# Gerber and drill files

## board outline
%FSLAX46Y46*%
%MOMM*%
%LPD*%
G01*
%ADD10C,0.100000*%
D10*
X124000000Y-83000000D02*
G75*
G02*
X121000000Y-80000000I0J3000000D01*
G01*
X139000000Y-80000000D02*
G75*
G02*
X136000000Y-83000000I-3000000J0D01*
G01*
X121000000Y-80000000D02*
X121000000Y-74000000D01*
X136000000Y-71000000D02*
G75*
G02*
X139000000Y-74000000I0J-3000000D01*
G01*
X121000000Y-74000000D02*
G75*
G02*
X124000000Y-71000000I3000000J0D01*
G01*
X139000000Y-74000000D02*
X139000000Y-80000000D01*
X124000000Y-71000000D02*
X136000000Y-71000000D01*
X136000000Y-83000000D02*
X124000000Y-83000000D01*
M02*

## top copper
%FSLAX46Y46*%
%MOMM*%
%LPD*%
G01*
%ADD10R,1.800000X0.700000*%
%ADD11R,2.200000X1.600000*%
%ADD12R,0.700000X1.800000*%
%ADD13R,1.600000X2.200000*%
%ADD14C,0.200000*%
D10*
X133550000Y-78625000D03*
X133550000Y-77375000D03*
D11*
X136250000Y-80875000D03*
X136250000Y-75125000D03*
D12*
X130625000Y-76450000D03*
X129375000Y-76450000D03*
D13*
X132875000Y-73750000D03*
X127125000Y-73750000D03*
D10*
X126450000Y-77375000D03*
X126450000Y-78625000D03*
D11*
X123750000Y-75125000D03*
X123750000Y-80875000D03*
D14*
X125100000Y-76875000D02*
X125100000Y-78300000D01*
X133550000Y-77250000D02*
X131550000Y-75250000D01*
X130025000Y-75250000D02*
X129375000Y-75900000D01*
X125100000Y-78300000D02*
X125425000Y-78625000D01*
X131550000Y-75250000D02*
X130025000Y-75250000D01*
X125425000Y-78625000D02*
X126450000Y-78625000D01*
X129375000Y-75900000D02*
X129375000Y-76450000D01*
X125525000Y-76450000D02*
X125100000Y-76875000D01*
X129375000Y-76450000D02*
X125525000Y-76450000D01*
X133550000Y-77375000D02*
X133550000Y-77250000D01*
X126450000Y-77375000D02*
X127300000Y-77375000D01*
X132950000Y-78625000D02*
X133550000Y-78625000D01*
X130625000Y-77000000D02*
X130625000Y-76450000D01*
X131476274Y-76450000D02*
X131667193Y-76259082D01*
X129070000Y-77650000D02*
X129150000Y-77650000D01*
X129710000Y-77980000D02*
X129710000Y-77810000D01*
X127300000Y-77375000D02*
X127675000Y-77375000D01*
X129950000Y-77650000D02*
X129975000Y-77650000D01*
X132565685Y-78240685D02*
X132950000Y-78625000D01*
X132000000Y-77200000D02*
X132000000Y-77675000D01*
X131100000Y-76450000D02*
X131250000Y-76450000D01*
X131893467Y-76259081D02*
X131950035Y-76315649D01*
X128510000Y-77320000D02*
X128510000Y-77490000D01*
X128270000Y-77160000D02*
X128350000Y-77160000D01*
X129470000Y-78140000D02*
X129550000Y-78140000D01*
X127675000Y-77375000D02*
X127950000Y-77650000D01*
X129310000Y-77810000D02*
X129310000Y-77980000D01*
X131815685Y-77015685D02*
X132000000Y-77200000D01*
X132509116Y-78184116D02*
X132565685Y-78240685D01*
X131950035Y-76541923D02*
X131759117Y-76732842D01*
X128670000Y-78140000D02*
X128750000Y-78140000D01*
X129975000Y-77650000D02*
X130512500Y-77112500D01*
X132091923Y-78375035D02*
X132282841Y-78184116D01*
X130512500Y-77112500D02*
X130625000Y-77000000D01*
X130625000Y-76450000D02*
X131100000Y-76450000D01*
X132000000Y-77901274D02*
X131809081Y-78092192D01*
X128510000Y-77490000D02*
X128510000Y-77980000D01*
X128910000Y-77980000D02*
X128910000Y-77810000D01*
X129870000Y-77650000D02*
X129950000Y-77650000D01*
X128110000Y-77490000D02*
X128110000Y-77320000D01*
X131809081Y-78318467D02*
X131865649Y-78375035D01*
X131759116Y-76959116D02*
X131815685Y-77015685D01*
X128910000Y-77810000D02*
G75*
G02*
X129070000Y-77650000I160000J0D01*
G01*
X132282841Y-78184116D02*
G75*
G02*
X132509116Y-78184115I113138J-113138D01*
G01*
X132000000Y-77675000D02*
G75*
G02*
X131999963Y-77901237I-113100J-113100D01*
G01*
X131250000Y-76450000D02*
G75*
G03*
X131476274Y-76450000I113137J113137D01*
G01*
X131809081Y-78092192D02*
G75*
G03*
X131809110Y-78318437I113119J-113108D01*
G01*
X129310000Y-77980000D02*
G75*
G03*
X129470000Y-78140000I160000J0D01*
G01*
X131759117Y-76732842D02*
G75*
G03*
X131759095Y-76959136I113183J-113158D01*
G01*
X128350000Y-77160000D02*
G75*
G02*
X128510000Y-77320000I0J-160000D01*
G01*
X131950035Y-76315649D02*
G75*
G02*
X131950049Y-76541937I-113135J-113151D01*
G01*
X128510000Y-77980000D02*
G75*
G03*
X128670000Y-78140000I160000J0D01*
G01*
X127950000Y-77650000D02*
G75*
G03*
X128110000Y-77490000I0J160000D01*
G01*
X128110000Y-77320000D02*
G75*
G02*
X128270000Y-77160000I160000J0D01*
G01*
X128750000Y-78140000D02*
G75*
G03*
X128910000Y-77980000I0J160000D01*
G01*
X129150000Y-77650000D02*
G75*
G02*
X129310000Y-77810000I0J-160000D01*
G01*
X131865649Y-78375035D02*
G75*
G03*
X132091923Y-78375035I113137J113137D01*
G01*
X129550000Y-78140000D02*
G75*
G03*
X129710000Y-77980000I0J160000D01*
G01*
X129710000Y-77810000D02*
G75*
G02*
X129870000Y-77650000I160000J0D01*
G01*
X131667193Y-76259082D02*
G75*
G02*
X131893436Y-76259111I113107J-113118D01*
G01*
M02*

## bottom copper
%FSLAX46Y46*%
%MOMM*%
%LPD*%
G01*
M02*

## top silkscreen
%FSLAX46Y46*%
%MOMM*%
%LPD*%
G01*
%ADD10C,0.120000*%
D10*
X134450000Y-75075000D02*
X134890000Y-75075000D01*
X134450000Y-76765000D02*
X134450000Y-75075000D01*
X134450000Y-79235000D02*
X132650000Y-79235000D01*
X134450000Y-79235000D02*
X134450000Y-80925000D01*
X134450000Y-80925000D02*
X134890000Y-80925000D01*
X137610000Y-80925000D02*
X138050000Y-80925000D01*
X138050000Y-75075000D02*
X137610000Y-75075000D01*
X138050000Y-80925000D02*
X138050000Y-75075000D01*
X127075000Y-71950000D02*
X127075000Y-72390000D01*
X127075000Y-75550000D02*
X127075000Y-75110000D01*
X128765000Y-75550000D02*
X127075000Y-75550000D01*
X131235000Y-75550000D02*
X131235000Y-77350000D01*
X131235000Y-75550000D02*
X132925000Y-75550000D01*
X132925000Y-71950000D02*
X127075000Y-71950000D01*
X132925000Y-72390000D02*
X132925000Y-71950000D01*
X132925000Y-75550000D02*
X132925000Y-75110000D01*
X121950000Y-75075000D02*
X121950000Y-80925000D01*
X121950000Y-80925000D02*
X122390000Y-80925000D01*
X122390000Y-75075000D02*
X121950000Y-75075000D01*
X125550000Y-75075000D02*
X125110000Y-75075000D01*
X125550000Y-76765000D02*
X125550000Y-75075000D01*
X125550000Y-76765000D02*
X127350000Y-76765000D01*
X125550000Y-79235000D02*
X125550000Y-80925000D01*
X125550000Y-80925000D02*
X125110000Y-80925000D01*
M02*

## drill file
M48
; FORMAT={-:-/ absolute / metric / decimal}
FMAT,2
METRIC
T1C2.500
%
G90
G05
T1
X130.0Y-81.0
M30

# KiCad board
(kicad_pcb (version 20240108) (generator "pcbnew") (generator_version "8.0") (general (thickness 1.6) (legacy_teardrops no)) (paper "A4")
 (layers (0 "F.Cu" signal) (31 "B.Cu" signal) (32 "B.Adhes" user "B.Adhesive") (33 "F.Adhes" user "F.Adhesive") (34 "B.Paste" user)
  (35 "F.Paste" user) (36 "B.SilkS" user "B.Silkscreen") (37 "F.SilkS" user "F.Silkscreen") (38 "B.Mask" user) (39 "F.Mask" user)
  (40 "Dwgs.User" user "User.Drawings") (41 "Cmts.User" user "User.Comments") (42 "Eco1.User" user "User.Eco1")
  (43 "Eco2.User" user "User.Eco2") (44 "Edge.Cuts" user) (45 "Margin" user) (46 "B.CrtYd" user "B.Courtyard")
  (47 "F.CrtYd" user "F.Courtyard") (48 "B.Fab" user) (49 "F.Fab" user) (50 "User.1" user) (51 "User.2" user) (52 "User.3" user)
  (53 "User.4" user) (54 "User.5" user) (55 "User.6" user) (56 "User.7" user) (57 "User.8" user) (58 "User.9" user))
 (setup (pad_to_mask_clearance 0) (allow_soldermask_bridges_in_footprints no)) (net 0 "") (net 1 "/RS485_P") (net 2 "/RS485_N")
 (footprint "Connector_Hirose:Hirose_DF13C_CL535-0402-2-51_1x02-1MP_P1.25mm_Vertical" (layer "F.Cu") (at 135 78 90)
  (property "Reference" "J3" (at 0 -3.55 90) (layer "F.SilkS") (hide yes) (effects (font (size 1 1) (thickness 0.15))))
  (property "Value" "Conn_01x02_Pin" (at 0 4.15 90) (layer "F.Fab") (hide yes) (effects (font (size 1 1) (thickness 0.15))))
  (fp_line (start 2.925 -0.55) (end 2.925 -0.11) (stroke (width 0.12) (type solid)) (layer "F.SilkS"))
  (fp_line (start 1.235 -0.55) (end 2.925 -0.55) (stroke (width 0.12) (type solid)) (layer "F.SilkS"))
  (fp_line (start -1.235 -0.55) (end -1.235 -2.35) (stroke (width 0.12) (type solid)) (layer "F.SilkS"))
  (fp_line (start -1.235 -0.55) (end -2.925 -0.55) (stroke (width 0.12) (type solid)) (layer "F.SilkS"))
  (fp_line (start -2.925 -0.55) (end -2.925 -0.11) (stroke (width 0.12) (type solid)) (layer "F.SilkS"))
  (fp_line (start -2.925 2.61) (end -2.925 3.05) (stroke (width 0.12) (type solid)) (layer "F.SilkS"))
  (fp_line (start 2.925 3.05) (end 2.925 2.61) (stroke (width 0.12) (type solid)) (layer "F.SilkS"))
  (fp_line (start -2.925 3.05) (end 2.925 3.05) (stroke (width 0.12) (type solid)) (layer "F.SilkS"))
  (pad "1" smd rect (at -0.625 -1.45 90) (size 0.7 1.8) (layers "F.Cu" "F.Paste" "F.Mask") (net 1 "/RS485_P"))
  (pad "2" smd rect (at 0.625 -1.45 90) (size 0.7 1.8) (layers "F.Cu" "F.Paste" "F.Mask") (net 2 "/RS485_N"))
  (pad "MP" smd rect (at -2.875 1.25 90) (size 1.6 2.2) (layers "F.Cu" "F.Paste" "F.Mask"))
  (pad "MP" smd rect (at 2.875 1.25 90) (size 1.6 2.2) (layers "F.Cu" "F.Paste" "F.Mask")))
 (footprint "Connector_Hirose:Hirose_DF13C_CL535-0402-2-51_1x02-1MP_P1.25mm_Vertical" (layer "F.Cu") (at 130 75 180)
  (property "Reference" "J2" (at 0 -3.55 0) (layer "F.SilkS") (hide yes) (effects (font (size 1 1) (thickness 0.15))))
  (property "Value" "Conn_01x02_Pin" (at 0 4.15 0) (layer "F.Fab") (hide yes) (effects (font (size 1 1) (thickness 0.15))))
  (fp_line (start 2.925 3.05) (end 2.925 2.61) (stroke (width 0.12) (type solid)) (layer "F.SilkS"))
  (fp_line (start 2.925 -0.55) (end 2.925 -0.11) (stroke (width 0.12) (type solid)) (layer "F.SilkS"))
  (fp_line (start 1.235 -0.55) (end 2.925 -0.55) (stroke (width 0.12) (type solid)) (layer "F.SilkS"))
  (fp_line (start -1.235 -0.55) (end -1.235 -2.35) (stroke (width 0.12) (type solid)) (layer "F.SilkS"))
  (fp_line (start -1.235 -0.55) (end -2.925 -0.55) (stroke (width 0.12) (type solid)) (layer "F.SilkS"))
  (fp_line (start -2.925 3.05) (end 2.925 3.05) (stroke (width 0.12) (type solid)) (layer "F.SilkS"))
  (fp_line (start -2.925 2.61) (end -2.925 3.05) (stroke (width 0.12) (type solid)) (layer "F.SilkS"))
  (fp_line (start -2.925 -0.55) (end -2.925 -0.11) (stroke (width 0.12) (type solid)) (layer "F.SilkS"))
  (pad "1" smd rect (at -0.625 -1.45 180) (size 0.7 1.8) (layers "F.Cu" "F.Paste" "F.Mask") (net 1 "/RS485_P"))
  (pad "2" smd rect (at 0.625 -1.45 180) (size 0.7 1.8) (layers "F.Cu" "F.Paste" "F.Mask") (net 2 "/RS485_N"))
  (pad "MP" smd rect (at -2.875 1.25 180) (size 1.6 2.2) (layers "F.Cu" "F.Paste" "F.Mask"))
  (pad "MP" smd rect (at 2.875 1.25 180) (size 1.6 2.2) (layers "F.Cu" "F.Paste" "F.Mask")))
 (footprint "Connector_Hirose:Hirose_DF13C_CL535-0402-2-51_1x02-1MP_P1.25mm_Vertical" (layer "F.Cu") (at 125 78 -90)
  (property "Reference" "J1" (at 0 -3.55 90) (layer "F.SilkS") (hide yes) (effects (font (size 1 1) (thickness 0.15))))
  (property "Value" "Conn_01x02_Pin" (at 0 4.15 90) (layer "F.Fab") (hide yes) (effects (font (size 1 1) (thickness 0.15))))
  (fp_line (start -2.925 3.05) (end 2.925 3.05) (stroke (width 0.12) (type solid)) (layer "F.SilkS"))
  (fp_line (start 2.925 3.05) (end 2.925 2.61) (stroke (width 0.12) (type solid)) (layer "F.SilkS"))
  (fp_line (start -2.925 2.61) (end -2.925 3.05) (stroke (width 0.12) (type solid)) (layer "F.SilkS"))
  (fp_line (start -2.925 -0.55) (end -2.925 -0.11) (stroke (width 0.12) (type solid)) (layer "F.SilkS"))
  (fp_line (start -1.235 -0.55) (end -2.925 -0.55) (stroke (width 0.12) (type solid)) (layer "F.SilkS"))
  (fp_line (start -1.235 -0.55) (end -1.235 -2.35) (stroke (width 0.12) (type solid)) (layer "F.SilkS"))
  (fp_line (start 1.235 -0.55) (end 2.925 -0.55) (stroke (width 0.12) (type solid)) (layer "F.SilkS"))
  (fp_line (start 2.925 -0.55) (end 2.925 -0.11) (stroke (width 0.12) (type solid)) (layer "F.SilkS"))
  (pad "1" smd rect (at -0.625 -1.45 270) (size 0.7 1.8) (layers "F.Cu" "F.Paste" "F.Mask") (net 1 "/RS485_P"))
  (pad "2" smd rect (at 0.625 -1.45 270) (size 0.7 1.8) (layers "F.Cu" "F.Paste" "F.Mask") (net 2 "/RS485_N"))
  (pad "MP" smd rect (at -2.875 1.25 270) (size 1.6 2.2) (layers "F.Cu" "F.Paste" "F.Mask"))
  (pad "MP" smd rect (at 2.875 1.25 270) (size 1.6 2.2) (layers "F.Cu" "F.Paste" "F.Mask")))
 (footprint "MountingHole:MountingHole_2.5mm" (layer "F.Cu") (at 130 81)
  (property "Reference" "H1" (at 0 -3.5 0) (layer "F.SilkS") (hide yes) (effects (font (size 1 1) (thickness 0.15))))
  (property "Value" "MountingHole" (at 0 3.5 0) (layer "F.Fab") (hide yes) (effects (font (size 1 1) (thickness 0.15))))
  (pad "" np_thru_hole circle (at 0 0) (size 2.5 2.5) (drill 2.5) (layers "*.Cu" "*.Mask")))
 (gr_arc (start 124 83) (mid 121.87868 82.12132) (end 121 80) (stroke (width 0.1) (type default)) (layer "Edge.Cuts"))
 (gr_arc (start 139 80) (mid 138.12132 82.12132) (end 136 83) (stroke (width 0.1) (type default)) (layer "Edge.Cuts"))
 (gr_line (start 121 80) (end 121 74) (stroke (width 0.1) (type default)) (layer "Edge.Cuts"))
 (gr_arc (start 136 71) (mid 138.12132 71.87868) (end 139 74) (stroke (width 0.1) (type default)) (layer "Edge.Cuts"))
 (gr_arc (start 121 74) (mid 121.87868 71.87868) (end 124 71) (stroke (width 0.1) (type default)) (layer "Edge.Cuts"))
 (gr_line (start 139 74) (end 139 80) (stroke (width 0.1) (type default)) (layer "Edge.Cuts"))
 (gr_line (start 124 71) (end 136 71) (stroke (width 0.1) (type default)) (layer "Edge.Cuts"))
 (gr_line (start 136 83) (end 124 83) (stroke (width 0.1) (type default)) (layer "Edge.Cuts"))
 (segment (start 125.1 76.875) (end 125.1 78.3) (width 0.2) (layer "F.Cu") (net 2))
 (segment (start 133.55 77.25) (end 131.55 75.25) (width 0.2) (layer "F.Cu") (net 2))
 (segment (start 130.025 75.25) (end 129.375 75.9) (width 0.2) (layer "F.Cu") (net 2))
 (segment (start 125.1 78.3) (end 125.425 78.625) (width 0.2) (layer "F.Cu") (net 2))
 (segment (start 131.55 75.25) (end 130.025 75.25) (width 0.2) (layer "F.Cu") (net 2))
 (segment (start 125.425 78.625) (end 126.45 78.625) (width 0.2) (layer "F.Cu") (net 2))
 (segment (start 129.375 75.9) (end 129.375 76.45) (width 0.2) (layer "F.Cu") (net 2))
 (segment (start 125.525 76.45) (end 125.1 76.875) (width 0.2) (layer "F.Cu") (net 2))
 (segment (start 129.375 76.45) (end 125.525 76.45) (width 0.2) (layer "F.Cu") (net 2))
 (segment (start 133.55 77.375) (end 133.55 77.25) (width 0.2) (layer "F.Cu") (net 2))
 (segment (start 126.45 77.375) (end 127.3 77.375) (width 0.2) (layer "F.Cu") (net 1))
 (segment (start 132.95 78.625) (end 133.55 78.625) (width 0.2) (layer "F.Cu") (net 1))
 (segment (start 130.625 77) (end 130.625 76.45) (width 0.2) (layer "F.Cu") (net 1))
 (segment (start 131.476274 76.45) (end 131.667193 76.259082) (width 0.2) (layer "F.Cu") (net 1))
 (segment (start 129.07 77.65) (end 129.15 77.65) (width 0.2) (layer "F.Cu") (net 1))
 (segment (start 129.71 77.98) (end 129.71 77.81) (width 0.2) (layer "F.Cu") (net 1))
 (segment (start 127.3 77.375) (end 127.675 77.375) (width 0.2) (layer "F.Cu") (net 1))
 (segment (start 129.95 77.65) (end 129.975 77.65) (width 0.2) (layer "F.Cu") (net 1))
 (segment (start 132.565685 78.240685) (end 132.95 78.625) (width 0.2) (layer "F.Cu") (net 1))
 (segment (start 132 77.2) (end 132 77.675) (width 0.2) (layer "F.Cu") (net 1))
 (segment (start 131.1 76.45) (end 131.25 76.45) (width 0.2) (layer "F.Cu") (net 1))
 (segment (start 131.893467 76.259081) (end 131.950035 76.315649) (width 0.2) (layer "F.Cu") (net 1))
 (segment (start 128.51 77.32) (end 128.51 77.49) (width 0.2) (layer "F.Cu") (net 1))
 (segment (start 128.27 77.16) (end 128.35 77.16) (width 0.2) (layer "F.Cu") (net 1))
 (segment (start 129.47 78.14) (end 129.55 78.14) (width 0.2) (layer "F.Cu") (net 1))
 (segment (start 127.675 77.375) (end 127.95 77.65) (width 0.2) (layer "F.Cu") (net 1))
 (segment (start 129.31 77.81) (end 129.31 77.98) (width 0.2) (layer "F.Cu") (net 1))
 (segment (start 131.815685 77.015685) (end 132 77.2) (width 0.2) (layer "F.Cu") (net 1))
 (segment (start 132.509116 78.184116) (end 132.565685 78.240685) (width 0.2) (layer "F.Cu") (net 1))
 (segment (start 131.950035 76.541923) (end 131.759117 76.732842) (width 0.2) (layer "F.Cu") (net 1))
 (segment (start 128.67 78.14) (end 128.75 78.14) (width 0.2) (layer "F.Cu") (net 1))
 (segment (start 129.975 77.65) (end 130.5125 77.1125) (width 0.2) (layer "F.Cu") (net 1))
 (segment (start 132.091923 78.375035) (end 132.282841 78.184116) (width 0.2) (layer "F.Cu") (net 1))
 (segment (start 130.5125 77.1125) (end 130.625 77) (width 0.2) (layer "F.Cu") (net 1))
 (segment (start 130.625 76.45) (end 131.1 76.45) (width 0.2) (layer "F.Cu") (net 1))
 (segment (start 132 77.901274) (end 131.809081 78.092192) (width 0.2) (layer "F.Cu") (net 1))
 (segment (start 128.51 77.49) (end 128.51 77.98) (width 0.2) (layer "F.Cu") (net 1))
 (segment (start 128.91 77.98) (end 128.91 77.81) (width 0.2) (layer "F.Cu") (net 1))
 (segment (start 129.87 77.65) (end 129.95 77.65) (width 0.2) (layer "F.Cu") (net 1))
 (segment (start 128.11 77.49) (end 128.11 77.32) (width 0.2) (layer "F.Cu") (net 1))
 (segment (start 131.809081 78.318467) (end 131.865649 78.375035) (width 0.2) (layer "F.Cu") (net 1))
 (segment (start 131.759116 76.959116) (end 131.815685 77.015685) (width 0.2) (layer "F.Cu") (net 1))
 (arc (start 128.91 77.81) (mid 128.956863 77.696863) (end 129.07 77.65) (width 0.2) (layer "F.Cu") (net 1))
 (arc (start 132.282841 78.184116) (mid 132.395978 78.137253) (end 132.509116 78.184116) (width 0.2) (layer "F.Cu") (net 1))
 (arc (start 132 77.675) (mid 132.046863 77.788137) (end 132 77.901274) (width 0.2) (layer "F.Cu") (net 1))
 (arc (start 131.25 76.45) (mid 131.363137 76.496863) (end 131.476274 76.45) (width 0.2) (layer "F.Cu") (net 1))
 (arc (start 131.809081 78.092192) (mid 131.762218 78.205329) (end 131.809081 78.318467) (width 0.2) (layer "F.Cu") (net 1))
 (arc (start 129.31 77.98) (mid 129.356863 78.093137) (end 129.47 78.14) (width 0.2) (layer "F.Cu") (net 1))
 (arc (start 131.759117 76.732842) (mid 131.712254 76.845979) (end 131.759116 76.959116) (width 0.2) (layer "F.Cu") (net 1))
 (arc (start 128.35 77.16) (mid 128.463137 77.206863) (end 128.51 77.32) (width 0.2) (layer "F.Cu") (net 1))
 (arc (start 131.950035 76.315649) (mid 131.996898 76.428786) (end 131.950035 76.541923) (width 0.2) (layer "F.Cu") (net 1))
 (arc (start 128.51 77.98) (mid 128.556863 78.093137) (end 128.67 78.14) (width 0.2) (layer "F.Cu") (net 1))
 (arc (start 127.95 77.65) (mid 128.063137 77.603137) (end 128.11 77.49) (width 0.2) (layer "F.Cu") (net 1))
 (arc (start 128.11 77.32) (mid 128.156863 77.206863) (end 128.27 77.16) (width 0.2) (layer "F.Cu") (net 1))
 (arc (start 128.75 78.14) (mid 128.863137 78.093137) (end 128.91 77.98) (width 0.2) (layer "F.Cu") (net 1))
 (arc (start 129.15 77.65) (mid 129.263137 77.696863) (end 129.31 77.81) (width 0.2) (layer "F.Cu") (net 1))
 (arc (start 131.865649 78.375035) (mid 131.978786 78.421898) (end 132.091923 78.375035) (width 0.2) (layer "F.Cu") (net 1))
 (arc (start 129.55 78.14) (mid 129.663137 78.093137) (end 129.71 77.98) (width 0.2) (layer "F.Cu") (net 1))
 (arc (start 129.71 77.81) (mid 129.756863 77.696863) (end 129.87 77.65) (width 0.2) (layer "F.Cu") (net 1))
 (arc (start 131.667193 76.259082) (mid 131.78033 76.212219) (end 131.893467 76.259081) (width 0.2) (layer "F.Cu") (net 1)))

